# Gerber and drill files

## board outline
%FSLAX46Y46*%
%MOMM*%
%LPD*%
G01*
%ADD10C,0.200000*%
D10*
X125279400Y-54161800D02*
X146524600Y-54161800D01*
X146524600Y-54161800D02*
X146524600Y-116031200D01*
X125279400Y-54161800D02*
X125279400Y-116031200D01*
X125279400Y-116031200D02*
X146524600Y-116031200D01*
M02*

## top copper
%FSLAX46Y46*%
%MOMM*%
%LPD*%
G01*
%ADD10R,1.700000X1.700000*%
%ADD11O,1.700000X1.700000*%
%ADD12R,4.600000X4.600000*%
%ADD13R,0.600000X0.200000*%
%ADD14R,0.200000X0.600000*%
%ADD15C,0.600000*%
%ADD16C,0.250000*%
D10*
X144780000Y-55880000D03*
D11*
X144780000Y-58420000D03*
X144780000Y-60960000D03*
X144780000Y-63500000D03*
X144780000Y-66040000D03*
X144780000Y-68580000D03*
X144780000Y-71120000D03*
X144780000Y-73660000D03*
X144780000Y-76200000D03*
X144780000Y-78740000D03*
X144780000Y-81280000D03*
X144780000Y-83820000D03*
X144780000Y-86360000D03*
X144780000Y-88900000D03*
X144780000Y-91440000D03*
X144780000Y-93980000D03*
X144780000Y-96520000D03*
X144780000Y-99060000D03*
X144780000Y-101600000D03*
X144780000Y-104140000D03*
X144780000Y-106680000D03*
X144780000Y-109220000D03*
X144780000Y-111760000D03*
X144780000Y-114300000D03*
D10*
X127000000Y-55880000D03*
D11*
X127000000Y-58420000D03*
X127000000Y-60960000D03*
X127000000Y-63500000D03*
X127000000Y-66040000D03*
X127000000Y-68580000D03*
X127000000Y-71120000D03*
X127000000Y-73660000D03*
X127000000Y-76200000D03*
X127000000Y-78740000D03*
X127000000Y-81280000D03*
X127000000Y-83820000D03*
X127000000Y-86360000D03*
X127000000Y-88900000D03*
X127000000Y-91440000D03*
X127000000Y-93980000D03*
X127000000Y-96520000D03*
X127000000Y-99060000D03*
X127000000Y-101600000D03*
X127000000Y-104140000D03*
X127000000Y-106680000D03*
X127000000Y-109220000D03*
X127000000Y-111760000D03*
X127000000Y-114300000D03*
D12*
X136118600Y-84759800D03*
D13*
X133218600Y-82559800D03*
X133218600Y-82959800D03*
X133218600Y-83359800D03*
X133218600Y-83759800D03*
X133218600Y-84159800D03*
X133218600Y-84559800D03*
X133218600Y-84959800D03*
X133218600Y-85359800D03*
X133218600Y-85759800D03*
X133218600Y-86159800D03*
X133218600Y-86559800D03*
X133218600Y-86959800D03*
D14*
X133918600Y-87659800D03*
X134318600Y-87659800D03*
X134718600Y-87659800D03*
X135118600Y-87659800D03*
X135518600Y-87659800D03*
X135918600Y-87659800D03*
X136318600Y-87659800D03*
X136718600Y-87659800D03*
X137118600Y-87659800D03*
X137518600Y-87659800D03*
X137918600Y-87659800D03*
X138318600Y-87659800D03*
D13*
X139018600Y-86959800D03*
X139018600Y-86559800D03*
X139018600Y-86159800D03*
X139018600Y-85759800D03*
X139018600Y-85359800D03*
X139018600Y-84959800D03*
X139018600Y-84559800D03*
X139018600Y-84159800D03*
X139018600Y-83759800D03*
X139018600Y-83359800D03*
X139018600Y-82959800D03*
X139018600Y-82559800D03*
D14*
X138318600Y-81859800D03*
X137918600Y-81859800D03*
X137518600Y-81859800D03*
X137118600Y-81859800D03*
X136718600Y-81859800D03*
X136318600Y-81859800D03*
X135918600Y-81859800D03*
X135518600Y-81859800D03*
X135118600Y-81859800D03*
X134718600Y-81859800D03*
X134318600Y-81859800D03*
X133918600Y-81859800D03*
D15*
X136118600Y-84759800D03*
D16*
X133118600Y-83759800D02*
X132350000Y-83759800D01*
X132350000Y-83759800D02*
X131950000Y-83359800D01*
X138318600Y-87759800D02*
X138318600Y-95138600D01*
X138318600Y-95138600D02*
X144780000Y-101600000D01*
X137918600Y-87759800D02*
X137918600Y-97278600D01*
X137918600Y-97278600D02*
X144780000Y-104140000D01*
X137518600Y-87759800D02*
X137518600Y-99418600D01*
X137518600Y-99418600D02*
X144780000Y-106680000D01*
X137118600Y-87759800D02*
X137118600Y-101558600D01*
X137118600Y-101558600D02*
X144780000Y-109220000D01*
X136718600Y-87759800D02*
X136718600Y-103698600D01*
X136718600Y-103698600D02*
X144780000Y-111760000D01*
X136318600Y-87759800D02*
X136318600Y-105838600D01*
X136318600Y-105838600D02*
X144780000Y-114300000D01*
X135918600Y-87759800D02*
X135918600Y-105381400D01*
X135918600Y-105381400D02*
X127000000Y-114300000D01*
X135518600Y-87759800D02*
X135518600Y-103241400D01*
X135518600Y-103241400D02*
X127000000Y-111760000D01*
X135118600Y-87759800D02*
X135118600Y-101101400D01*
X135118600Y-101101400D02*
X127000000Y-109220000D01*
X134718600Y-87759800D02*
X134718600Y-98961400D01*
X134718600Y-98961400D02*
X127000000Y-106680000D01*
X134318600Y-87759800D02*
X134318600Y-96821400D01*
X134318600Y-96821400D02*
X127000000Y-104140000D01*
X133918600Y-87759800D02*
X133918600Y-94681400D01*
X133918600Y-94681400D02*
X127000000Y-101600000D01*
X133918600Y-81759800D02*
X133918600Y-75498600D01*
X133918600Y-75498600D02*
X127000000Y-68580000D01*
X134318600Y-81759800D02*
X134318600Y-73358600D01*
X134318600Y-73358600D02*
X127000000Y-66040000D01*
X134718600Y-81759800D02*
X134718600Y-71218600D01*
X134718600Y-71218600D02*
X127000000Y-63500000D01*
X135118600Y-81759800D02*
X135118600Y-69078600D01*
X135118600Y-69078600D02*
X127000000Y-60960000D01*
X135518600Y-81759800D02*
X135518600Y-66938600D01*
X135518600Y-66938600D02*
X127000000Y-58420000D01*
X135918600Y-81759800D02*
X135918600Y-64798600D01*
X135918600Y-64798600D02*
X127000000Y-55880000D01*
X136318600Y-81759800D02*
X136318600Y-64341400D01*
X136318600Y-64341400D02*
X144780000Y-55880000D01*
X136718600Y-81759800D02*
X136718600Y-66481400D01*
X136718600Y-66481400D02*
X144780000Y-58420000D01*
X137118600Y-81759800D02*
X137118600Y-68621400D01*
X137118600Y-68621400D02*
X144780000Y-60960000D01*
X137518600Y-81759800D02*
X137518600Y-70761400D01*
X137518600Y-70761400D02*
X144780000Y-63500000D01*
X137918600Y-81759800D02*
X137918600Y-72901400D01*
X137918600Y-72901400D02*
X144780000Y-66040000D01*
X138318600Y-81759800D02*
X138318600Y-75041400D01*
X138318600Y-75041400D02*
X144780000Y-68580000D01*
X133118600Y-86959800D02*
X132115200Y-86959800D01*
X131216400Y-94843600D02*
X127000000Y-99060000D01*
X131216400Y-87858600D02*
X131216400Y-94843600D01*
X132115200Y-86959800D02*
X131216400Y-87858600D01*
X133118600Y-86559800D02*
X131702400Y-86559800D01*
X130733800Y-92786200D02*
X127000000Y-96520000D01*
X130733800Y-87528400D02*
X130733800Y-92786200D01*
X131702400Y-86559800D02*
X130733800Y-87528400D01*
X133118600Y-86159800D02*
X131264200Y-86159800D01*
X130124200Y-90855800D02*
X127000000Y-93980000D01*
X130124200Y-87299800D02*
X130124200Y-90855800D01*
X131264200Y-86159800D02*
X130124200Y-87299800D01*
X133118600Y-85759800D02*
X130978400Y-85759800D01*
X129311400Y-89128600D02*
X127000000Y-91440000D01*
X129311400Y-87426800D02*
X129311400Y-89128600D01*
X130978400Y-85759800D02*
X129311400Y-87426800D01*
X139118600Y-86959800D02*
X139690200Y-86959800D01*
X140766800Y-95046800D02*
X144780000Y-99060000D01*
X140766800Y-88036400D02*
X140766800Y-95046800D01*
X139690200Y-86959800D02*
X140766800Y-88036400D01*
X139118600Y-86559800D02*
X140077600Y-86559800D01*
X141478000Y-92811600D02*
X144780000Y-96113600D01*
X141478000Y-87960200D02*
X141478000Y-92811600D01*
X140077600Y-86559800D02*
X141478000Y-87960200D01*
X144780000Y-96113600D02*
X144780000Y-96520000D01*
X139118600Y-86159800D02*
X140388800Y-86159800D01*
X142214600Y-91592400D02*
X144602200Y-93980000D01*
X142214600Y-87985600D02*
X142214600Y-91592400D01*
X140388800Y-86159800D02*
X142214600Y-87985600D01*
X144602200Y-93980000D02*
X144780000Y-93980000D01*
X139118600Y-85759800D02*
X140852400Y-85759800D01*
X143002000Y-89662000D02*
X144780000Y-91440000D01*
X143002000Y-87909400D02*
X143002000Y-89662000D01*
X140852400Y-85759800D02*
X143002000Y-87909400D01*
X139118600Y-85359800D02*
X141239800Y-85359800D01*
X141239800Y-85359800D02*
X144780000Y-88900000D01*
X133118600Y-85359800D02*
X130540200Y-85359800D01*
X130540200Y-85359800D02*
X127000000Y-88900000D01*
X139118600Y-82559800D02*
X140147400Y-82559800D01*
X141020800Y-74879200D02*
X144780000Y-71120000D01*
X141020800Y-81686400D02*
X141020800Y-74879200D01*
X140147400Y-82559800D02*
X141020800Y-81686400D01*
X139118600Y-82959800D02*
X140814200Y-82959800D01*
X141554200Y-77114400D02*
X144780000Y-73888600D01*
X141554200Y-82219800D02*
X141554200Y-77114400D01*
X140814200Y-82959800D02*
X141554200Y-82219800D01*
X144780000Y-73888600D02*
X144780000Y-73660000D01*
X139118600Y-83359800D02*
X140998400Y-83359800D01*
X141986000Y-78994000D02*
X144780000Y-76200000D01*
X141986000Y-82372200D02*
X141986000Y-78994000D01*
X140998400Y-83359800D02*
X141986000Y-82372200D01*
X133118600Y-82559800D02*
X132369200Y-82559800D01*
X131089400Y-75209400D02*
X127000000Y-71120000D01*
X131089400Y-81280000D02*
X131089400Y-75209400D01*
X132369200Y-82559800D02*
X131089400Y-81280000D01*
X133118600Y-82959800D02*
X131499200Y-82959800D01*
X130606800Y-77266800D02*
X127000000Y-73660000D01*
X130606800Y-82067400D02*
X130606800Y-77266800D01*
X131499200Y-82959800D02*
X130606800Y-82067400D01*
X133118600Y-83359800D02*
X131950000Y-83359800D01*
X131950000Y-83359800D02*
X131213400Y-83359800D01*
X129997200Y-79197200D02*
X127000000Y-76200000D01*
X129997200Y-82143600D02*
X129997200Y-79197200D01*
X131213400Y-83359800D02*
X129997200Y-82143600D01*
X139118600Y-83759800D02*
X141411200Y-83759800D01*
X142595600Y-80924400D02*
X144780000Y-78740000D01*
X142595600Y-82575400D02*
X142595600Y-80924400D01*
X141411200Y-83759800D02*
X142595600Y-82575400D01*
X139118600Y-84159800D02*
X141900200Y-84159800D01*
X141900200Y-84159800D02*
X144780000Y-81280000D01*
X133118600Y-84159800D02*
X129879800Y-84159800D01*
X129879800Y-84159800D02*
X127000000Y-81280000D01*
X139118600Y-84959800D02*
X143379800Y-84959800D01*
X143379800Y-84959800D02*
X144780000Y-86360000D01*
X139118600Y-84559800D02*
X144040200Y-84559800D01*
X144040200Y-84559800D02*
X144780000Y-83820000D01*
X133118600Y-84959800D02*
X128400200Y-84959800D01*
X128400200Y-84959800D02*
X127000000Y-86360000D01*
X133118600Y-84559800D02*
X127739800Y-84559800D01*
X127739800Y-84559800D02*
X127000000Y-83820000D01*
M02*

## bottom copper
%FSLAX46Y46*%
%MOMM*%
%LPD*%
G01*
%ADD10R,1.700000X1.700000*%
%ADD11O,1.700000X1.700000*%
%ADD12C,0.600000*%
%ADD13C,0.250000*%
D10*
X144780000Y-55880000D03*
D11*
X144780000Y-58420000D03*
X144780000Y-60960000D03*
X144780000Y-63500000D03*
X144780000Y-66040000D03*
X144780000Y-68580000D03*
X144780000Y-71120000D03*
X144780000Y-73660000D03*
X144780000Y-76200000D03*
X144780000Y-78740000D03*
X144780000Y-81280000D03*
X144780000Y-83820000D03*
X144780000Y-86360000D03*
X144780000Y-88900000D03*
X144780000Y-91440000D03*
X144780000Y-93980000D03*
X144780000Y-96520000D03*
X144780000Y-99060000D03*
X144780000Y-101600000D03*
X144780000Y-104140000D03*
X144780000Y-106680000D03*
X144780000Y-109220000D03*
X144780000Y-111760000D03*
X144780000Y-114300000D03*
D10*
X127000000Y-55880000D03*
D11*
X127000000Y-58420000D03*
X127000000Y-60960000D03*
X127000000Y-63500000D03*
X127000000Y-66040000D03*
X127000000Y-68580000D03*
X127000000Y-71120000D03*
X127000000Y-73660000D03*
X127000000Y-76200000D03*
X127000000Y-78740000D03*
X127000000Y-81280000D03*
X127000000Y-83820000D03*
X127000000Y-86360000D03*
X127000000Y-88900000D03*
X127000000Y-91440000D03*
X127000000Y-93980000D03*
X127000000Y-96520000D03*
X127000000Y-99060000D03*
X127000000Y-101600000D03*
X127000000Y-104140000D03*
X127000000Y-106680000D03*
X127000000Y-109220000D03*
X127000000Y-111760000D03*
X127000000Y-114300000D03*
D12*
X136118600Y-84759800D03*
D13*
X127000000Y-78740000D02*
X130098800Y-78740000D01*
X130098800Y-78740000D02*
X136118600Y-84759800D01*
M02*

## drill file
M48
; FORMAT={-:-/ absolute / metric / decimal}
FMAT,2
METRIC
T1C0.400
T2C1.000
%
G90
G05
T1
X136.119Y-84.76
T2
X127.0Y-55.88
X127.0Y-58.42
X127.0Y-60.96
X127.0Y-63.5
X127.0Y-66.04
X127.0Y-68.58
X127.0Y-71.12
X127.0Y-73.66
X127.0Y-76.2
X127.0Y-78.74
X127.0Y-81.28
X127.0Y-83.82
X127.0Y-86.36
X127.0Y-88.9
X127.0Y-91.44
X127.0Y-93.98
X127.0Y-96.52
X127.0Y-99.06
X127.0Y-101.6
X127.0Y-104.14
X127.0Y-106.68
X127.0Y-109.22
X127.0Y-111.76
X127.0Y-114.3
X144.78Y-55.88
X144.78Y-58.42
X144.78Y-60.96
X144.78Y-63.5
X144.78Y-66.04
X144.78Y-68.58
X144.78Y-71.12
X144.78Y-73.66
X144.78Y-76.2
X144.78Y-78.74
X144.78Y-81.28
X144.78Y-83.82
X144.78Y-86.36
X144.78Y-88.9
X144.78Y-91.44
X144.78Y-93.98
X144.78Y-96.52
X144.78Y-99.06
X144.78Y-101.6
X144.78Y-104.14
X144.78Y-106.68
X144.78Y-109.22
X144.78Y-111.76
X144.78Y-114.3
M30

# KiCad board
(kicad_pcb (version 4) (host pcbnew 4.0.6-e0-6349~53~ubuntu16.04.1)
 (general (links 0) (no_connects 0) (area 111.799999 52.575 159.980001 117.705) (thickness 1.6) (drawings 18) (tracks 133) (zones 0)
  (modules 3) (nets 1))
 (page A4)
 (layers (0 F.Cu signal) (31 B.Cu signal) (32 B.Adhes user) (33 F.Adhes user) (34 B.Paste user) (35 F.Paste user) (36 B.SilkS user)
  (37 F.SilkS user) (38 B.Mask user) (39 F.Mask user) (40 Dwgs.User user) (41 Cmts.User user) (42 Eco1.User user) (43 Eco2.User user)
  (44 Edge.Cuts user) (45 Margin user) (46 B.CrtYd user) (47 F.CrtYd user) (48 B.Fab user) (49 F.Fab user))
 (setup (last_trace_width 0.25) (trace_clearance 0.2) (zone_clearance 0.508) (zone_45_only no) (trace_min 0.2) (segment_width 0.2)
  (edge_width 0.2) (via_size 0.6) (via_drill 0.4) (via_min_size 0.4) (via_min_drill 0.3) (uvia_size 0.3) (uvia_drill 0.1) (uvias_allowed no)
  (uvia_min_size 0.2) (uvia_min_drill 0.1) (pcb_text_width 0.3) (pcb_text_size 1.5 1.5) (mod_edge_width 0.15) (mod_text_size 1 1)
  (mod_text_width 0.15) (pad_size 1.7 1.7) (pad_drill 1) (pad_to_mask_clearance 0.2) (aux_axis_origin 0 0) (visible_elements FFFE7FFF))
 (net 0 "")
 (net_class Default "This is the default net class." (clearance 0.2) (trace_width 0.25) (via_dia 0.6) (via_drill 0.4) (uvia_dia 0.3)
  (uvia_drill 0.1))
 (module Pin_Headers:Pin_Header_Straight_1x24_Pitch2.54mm (layer F.Cu) (at 144.78 55.88)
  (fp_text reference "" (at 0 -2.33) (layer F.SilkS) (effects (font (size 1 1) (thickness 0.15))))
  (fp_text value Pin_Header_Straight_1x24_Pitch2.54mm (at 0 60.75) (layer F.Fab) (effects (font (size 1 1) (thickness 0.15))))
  (pad 1 thru_hole rect (at 0 0) (size 1.7 1.7) (drill 1) (layers *.Cu *.Mask))
  (pad 2 thru_hole oval (at 0 2.54) (size 1.7 1.7) (drill 1) (layers *.Cu *.Mask))
  (pad 3 thru_hole oval (at 0 5.08) (size 1.7 1.7) (drill 1) (layers *.Cu *.Mask))
  (pad 4 thru_hole oval (at 0 7.62) (size 1.7 1.7) (drill 1) (layers *.Cu *.Mask))
  (pad 5 thru_hole oval (at 0 10.16) (size 1.7 1.7) (drill 1) (layers *.Cu *.Mask))
  (pad 6 thru_hole oval (at 0 12.7) (size 1.7 1.7) (drill 1) (layers *.Cu *.Mask))
  (pad 7 thru_hole oval (at 0 15.24) (size 1.7 1.7) (drill 1) (layers *.Cu *.Mask))
  (pad 8 thru_hole oval (at 0 17.78) (size 1.7 1.7) (drill 1) (layers *.Cu *.Mask))
  (pad 9 thru_hole oval (at 0 20.32) (size 1.7 1.7) (drill 1) (layers *.Cu *.Mask))
  (pad 10 thru_hole oval (at 0 22.86) (size 1.7 1.7) (drill 1) (layers *.Cu *.Mask))
  (pad 11 thru_hole oval (at 0 25.4) (size 1.7 1.7) (drill 1) (layers *.Cu *.Mask))
  (pad 12 thru_hole oval (at 0 27.94) (size 1.7 1.7) (drill 1) (layers *.Cu *.Mask))
  (pad 13 thru_hole oval (at 0 30.48) (size 1.7 1.7) (drill 1) (layers *.Cu *.Mask))
  (pad 14 thru_hole oval (at 0 33.02) (size 1.7 1.7) (drill 1) (layers *.Cu *.Mask))
  (pad 15 thru_hole oval (at 0 35.56) (size 1.7 1.7) (drill 1) (layers *.Cu *.Mask))
  (pad 16 thru_hole oval (at 0 38.1) (size 1.7 1.7) (drill 1) (layers *.Cu *.Mask))
  (pad 17 thru_hole oval (at 0 40.64) (size 1.7 1.7) (drill 1) (layers *.Cu *.Mask))
  (pad 18 thru_hole oval (at 0 43.18) (size 1.7 1.7) (drill 1) (layers *.Cu *.Mask))
  (pad 19 thru_hole oval (at 0 45.72) (size 1.7 1.7) (drill 1) (layers *.Cu *.Mask))
  (pad 20 thru_hole oval (at 0 48.26) (size 1.7 1.7) (drill 1) (layers *.Cu *.Mask))
  (pad 21 thru_hole oval (at 0 50.8) (size 1.7 1.7) (drill 1) (layers *.Cu *.Mask))
  (pad 22 thru_hole oval (at 0 53.34) (size 1.7 1.7) (drill 1) (layers *.Cu *.Mask))
  (pad 23 thru_hole oval (at 0 55.88) (size 1.7 1.7) (drill 1) (layers *.Cu *.Mask))
  (pad 24 thru_hole oval (at 0 58.42) (size 1.7 1.7) (drill 1) (layers *.Cu *.Mask)))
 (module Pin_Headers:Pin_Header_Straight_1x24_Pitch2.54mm (layer F.Cu) (at 127 55.88)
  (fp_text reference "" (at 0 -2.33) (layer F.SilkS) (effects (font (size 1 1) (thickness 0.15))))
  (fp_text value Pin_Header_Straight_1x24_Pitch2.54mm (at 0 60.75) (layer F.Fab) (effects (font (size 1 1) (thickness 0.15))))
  (pad 1 thru_hole rect (at 0 0) (size 1.7 1.7) (drill 1) (layers *.Cu *.Mask))
  (pad 2 thru_hole oval (at 0 2.54) (size 1.7 1.7) (drill 1) (layers *.Cu *.Mask))
  (pad 3 thru_hole oval (at 0 5.08) (size 1.7 1.7) (drill 1) (layers *.Cu *.Mask))
  (pad 4 thru_hole oval (at 0 7.62) (size 1.7 1.7) (drill 1) (layers *.Cu *.Mask))
  (pad 5 thru_hole oval (at 0 10.16) (size 1.7 1.7) (drill 1) (layers *.Cu *.Mask))
  (pad 6 thru_hole oval (at 0 12.7) (size 1.7 1.7) (drill 1) (layers *.Cu *.Mask))
  (pad 7 thru_hole oval (at 0 15.24) (size 1.7 1.7) (drill 1) (layers *.Cu *.Mask))
  (pad 8 thru_hole oval (at 0 17.78) (size 1.7 1.7) (drill 1) (layers *.Cu *.Mask))
  (pad 9 thru_hole oval (at 0 20.32) (size 1.7 1.7) (drill 1) (layers *.Cu *.Mask))
  (pad 10 thru_hole oval (at 0 22.86) (size 1.7 1.7) (drill 1) (layers *.Cu *.Mask))
  (pad 11 thru_hole oval (at 0 25.4) (size 1.7 1.7) (drill 1) (layers *.Cu *.Mask))
  (pad 12 thru_hole oval (at 0 27.94) (size 1.7 1.7) (drill 1) (layers *.Cu *.Mask))
  (pad 13 thru_hole oval (at 0 30.48) (size 1.7 1.7) (drill 1) (layers *.Cu *.Mask))
  (pad 14 thru_hole oval (at 0 33.02) (size 1.7 1.7) (drill 1) (layers *.Cu *.Mask))
  (pad 15 thru_hole oval (at 0 35.56) (size 1.7 1.7) (drill 1) (layers *.Cu *.Mask))
  (pad 16 thru_hole oval (at 0 38.1) (size 1.7 1.7) (drill 1) (layers *.Cu *.Mask))
  (pad 17 thru_hole oval (at 0 40.64) (size 1.7 1.7) (drill 1) (layers *.Cu *.Mask))
  (pad 18 thru_hole oval (at 0 43.18) (size 1.7 1.7) (drill 1) (layers *.Cu *.Mask))
  (pad 19 thru_hole oval (at 0 45.72) (size 1.7 1.7) (drill 1) (layers *.Cu *.Mask))
  (pad 20 thru_hole oval (at 0 48.26) (size 1.7 1.7) (drill 1) (layers *.Cu *.Mask))
  (pad 21 thru_hole oval (at 0 50.8) (size 1.7 1.7) (drill 1) (layers *.Cu *.Mask))
  (pad 22 thru_hole oval (at 0 53.34) (size 1.7 1.7) (drill 1) (layers *.Cu *.Mask))
  (pad 23 thru_hole oval (at 0 55.88) (size 1.7 1.7) (drill 1) (layers *.Cu *.Mask))
  (pad 24 thru_hole oval (at 0 58.42) (size 1.7 1.7) (drill 1) (layers *.Cu *.Mask)))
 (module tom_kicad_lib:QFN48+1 (layer F.Cu) (at 136.1186 84.7598) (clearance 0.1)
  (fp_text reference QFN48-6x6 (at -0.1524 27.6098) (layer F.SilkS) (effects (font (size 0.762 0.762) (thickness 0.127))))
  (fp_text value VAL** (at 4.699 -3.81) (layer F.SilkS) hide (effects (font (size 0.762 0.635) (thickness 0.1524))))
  (pad 49 smd rect (at 0 0) (size 4.6 4.6) (layers F.Cu F.Paste F.Mask))
  (pad 1 smd rect (at -3 -2.2) (size 0.6 0.2) (drill (offset 0.1 0)) (layers F.Cu F.Paste F.Mask))
  (pad 2 smd rect (at -3 -1.8) (size 0.6 0.2) (drill (offset 0.1 0)) (layers F.Cu F.Paste F.Mask))
  (pad 3 smd rect (at -3 -1.4) (size 0.6 0.2) (drill (offset 0.1 0)) (layers F.Cu F.Paste F.Mask))
  (pad 4 smd rect (at -3 -1) (size 0.6 0.2) (drill (offset 0.1 0)) (layers F.Cu F.Paste F.Mask))
  (pad 5 smd rect (at -3 -0.6) (size 0.6 0.2) (drill (offset 0.1 0)) (layers F.Cu F.Paste F.Mask))
  (pad 6 smd rect (at -3 -0.2) (size 0.6 0.2) (drill (offset 0.1 0)) (layers F.Cu F.Paste F.Mask))
  (pad 7 smd rect (at -3 0.2) (size 0.6 0.2) (drill (offset 0.1 0)) (layers F.Cu F.Paste F.Mask))
  (pad 8 smd rect (at -3 0.6) (size 0.6 0.2) (drill (offset 0.1 0)) (layers F.Cu F.Paste F.Mask))
  (pad 9 smd rect (at -3 1) (size 0.6 0.2) (drill (offset 0.1 0)) (layers F.Cu F.Paste F.Mask))
  (pad 10 smd rect (at -3 1.4) (size 0.6 0.2) (drill (offset 0.1 0)) (layers F.Cu F.Paste F.Mask))
  (pad 11 smd rect (at -3 1.8) (size 0.6 0.2) (drill (offset 0.1 0)) (layers F.Cu F.Paste F.Mask))
  (pad 12 smd rect (at -3 2.2) (size 0.6 0.2) (drill (offset 0.1 0)) (layers F.Cu F.Paste F.Mask))
  (pad 13 smd rect (at -2.2 3 90) (size 0.6 0.2) (drill (offset 0.1 0)) (layers F.Cu F.Paste F.Mask))
  (pad 14 smd rect (at -1.8 3 90) (size 0.6 0.2) (drill (offset 0.1 0)) (layers F.Cu F.Paste F.Mask))
  (pad 15 smd rect (at -1.4 3 90) (size 0.6 0.2) (drill (offset 0.1 0)) (layers F.Cu F.Paste F.Mask))
  (pad 16 smd rect (at -1 3 90) (size 0.6 0.2) (drill (offset 0.1 0)) (layers F.Cu F.Paste F.Mask))
  (pad 17 smd rect (at -0.6 3 90) (size 0.6 0.2) (drill (offset 0.1 0)) (layers F.Cu F.Paste F.Mask))
  (pad 18 smd rect (at -0.2 3 90) (size 0.6 0.2) (drill (offset 0.1 0)) (layers F.Cu F.Paste F.Mask))
  (pad 19 smd rect (at 0.2 3 90) (size 0.6 0.2) (drill (offset 0.1 0)) (layers F.Cu F.Paste F.Mask))
  (pad 20 smd rect (at 0.6 3 90) (size 0.6 0.2) (drill (offset 0.1 0)) (layers F.Cu F.Paste F.Mask))
  (pad 21 smd rect (at 1 3 90) (size 0.6 0.2) (drill (offset 0.1 0)) (layers F.Cu F.Paste F.Mask))
  (pad 22 smd rect (at 1.4 3 90) (size 0.6 0.2) (drill (offset 0.1 0)) (layers F.Cu F.Paste F.Mask))
  (pad 23 smd rect (at 1.8 3 90) (size 0.6 0.2) (drill (offset 0.1 0)) (layers F.Cu F.Paste F.Mask))
  (pad 24 smd rect (at 2.2 3 90) (size 0.6 0.2) (drill (offset 0.1 0)) (layers F.Cu F.Paste F.Mask))
  (pad 25 smd rect (at 3 2.2 180) (size 0.6 0.2) (drill (offset 0.1 0)) (layers F.Cu F.Paste F.Mask))
  (pad 26 smd rect (at 3 1.8 180) (size 0.6 0.2) (drill (offset 0.1 0)) (layers F.Cu F.Paste F.Mask))
  (pad 27 smd rect (at 3 1.4 180) (size 0.6 0.2) (drill (offset 0.1 0)) (layers F.Cu F.Paste F.Mask))
  (pad 28 smd rect (at 3 1 180) (size 0.6 0.2) (drill (offset 0.1 0)) (layers F.Cu F.Paste F.Mask))
  (pad 29 smd rect (at 3 0.6 180) (size 0.6 0.2) (drill (offset 0.1 0)) (layers F.Cu F.Paste F.Mask))
  (pad 30 smd rect (at 3 0.2 180) (size 0.6 0.2) (drill (offset 0.1 0)) (layers F.Cu F.Paste F.Mask))
  (pad 31 smd rect (at 3 -0.2 180) (size 0.6 0.2) (drill (offset 0.1 0)) (layers F.Cu F.Paste F.Mask))
  (pad 32 smd rect (at 3 -0.6 180) (size 0.6 0.2) (drill (offset 0.1 0)) (layers F.Cu F.Paste F.Mask))
  (pad 33 smd rect (at 3 -1 180) (size 0.6 0.2) (drill (offset 0.1 0)) (layers F.Cu F.Paste F.Mask))
  (pad 34 smd rect (at 3 -1.4 180) (size 0.6 0.2) (drill (offset 0.1 0)) (layers F.Cu F.Paste F.Mask))
  (pad 35 smd rect (at 3 -1.8 180) (size 0.6 0.2) (drill (offset 0.1 0)) (layers F.Cu F.Paste F.Mask))
  (pad 36 smd rect (at 3 -2.2 180) (size 0.6 0.2) (drill (offset 0.1 0)) (layers F.Cu F.Paste F.Mask))
  (pad 37 smd rect (at 2.2 -3 270) (size 0.6 0.2) (drill (offset 0.1 0)) (layers F.Cu F.Paste F.Mask))
  (pad 38 smd rect (at 1.8 -3 270) (size 0.6 0.2) (drill (offset 0.1 0)) (layers F.Cu F.Paste F.Mask))
  (pad 39 smd rect (at 1.4 -3 270) (size 0.6 0.2) (drill (offset 0.1 0)) (layers F.Cu F.Paste F.Mask))
  (pad 40 smd rect (at 1 -3 270) (size 0.6 0.2) (drill (offset 0.1 0)) (layers F.Cu F.Paste F.Mask))
  (pad 41 smd rect (at 0.6 -3 270) (size 0.6 0.2) (drill (offset 0.1 0)) (layers F.Cu F.Paste F.Mask))
  (pad 42 smd rect (at 0.2 -3 270) (size 0.6 0.2) (drill (offset 0.1 0)) (layers F.Cu F.Paste F.Mask))
  (pad 43 smd rect (at -0.2 -3 270) (size 0.6 0.2) (drill (offset 0.1 0)) (layers F.Cu F.Paste F.Mask))
  (pad 44 smd rect (at -0.6 -3 270) (size 0.6 0.2) (drill (offset 0.1 0)) (layers F.Cu F.Paste F.Mask))
  (pad 45 smd rect (at -1 -3 270) (size 0.6 0.2) (drill (offset 0.1 0)) (layers F.Cu F.Paste F.Mask))
  (pad 46 smd rect (at -1.4 -3 270) (size 0.6 0.2) (drill (offset 0.1 0)) (layers F.Cu F.Paste F.Mask))
  (pad 47 smd rect (at -1.8 -3 270) (size 0.6 0.2) (drill (offset 0.1 0)) (layers F.Cu F.Paste F.Mask))
  (pad 48 smd rect (at -2.2 -3 270) (size 0.6 0.2) (drill (offset 0.1 0)) (layers F.Cu F.Paste F.Mask)))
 (gr_line (start 125.2794 54.1618) (end 146.5246 54.1618) (angle 90) (layer Edge.Cuts) (width 0.2))
 (gr_line (start 146.5246 54.1618) (end 146.5246 116.0312) (angle 90) (layer Edge.Cuts) (width 0.2))
 (gr_line (start 125.2794 54.1618) (end 125.2794 116.0312) (angle 90) (layer Edge.Cuts) (width 0.2))
 (gr_line (start 125.2794 116.0312) (end 146.5246 116.0312) (angle 90) (layer Edge.Cuts) (width 0.2))
 (via (at 136.1186 84.7598) (size 0.6) (drill 0.4) (layers F.Cu B.Cu) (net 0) (status C00000))
 (segment (start 127 78.74) (end 130.0988 78.74) (width 0.25) (layer B.Cu) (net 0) (status 400000))
 (segment (start 130.0988 78.74) (end 136.1186 84.7598) (width 0.25) (layer B.Cu) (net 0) (status 800000))
 (segment (start 133.1186 83.7598) (end 132.35 83.7598) (width 0.25) (layer F.Cu) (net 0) (status 400000))
 (segment (start 132.35 83.7598) (end 131.95 83.3598) (width 0.25) (layer F.Cu) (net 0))
 (segment (start 138.3186 87.7598) (end 138.3186 95.1386) (width 0.25) (layer F.Cu) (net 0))
 (segment (start 138.3186 95.1386) (end 144.78 101.6) (width 0.25) (layer F.Cu) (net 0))
 (segment (start 137.9186 87.7598) (end 137.9186 97.2786) (width 0.25) (layer F.Cu) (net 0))
 (segment (start 137.9186 97.2786) (end 144.78 104.14) (width 0.25) (layer F.Cu) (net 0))
 (segment (start 137.5186 87.7598) (end 137.5186 99.4186) (width 0.25) (layer F.Cu) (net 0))
 (segment (start 137.5186 99.4186) (end 144.78 106.68) (width 0.25) (layer F.Cu) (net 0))
 (segment (start 137.1186 87.7598) (end 137.1186 101.5586) (width 0.25) (layer F.Cu) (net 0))
 (segment (start 137.1186 101.5586) (end 144.78 109.22) (width 0.25) (layer F.Cu) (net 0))
 (segment (start 136.7186 87.7598) (end 136.7186 103.6986) (width 0.25) (layer F.Cu) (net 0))
 (segment (start 136.7186 103.6986) (end 144.78 111.76) (width 0.25) (layer F.Cu) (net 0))
 (segment (start 136.3186 87.7598) (end 136.3186 105.8386) (width 0.25) (layer F.Cu) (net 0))
 (segment (start 136.3186 105.8386) (end 144.78 114.3) (width 0.25) (layer F.Cu) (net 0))
 (segment (start 135.9186 87.7598) (end 135.9186 105.3814) (width 0.25) (layer F.Cu) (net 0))
 (segment (start 135.9186 105.3814) (end 127 114.3) (width 0.25) (layer F.Cu) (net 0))
 (segment (start 135.5186 87.7598) (end 135.5186 103.2414) (width 0.25) (layer F.Cu) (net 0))
 (segment (start 135.5186 103.2414) (end 127 111.76) (width 0.25) (layer F.Cu) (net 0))
 (segment (start 135.1186 87.7598) (end 135.1186 101.1014) (width 0.25) (layer F.Cu) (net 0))
 (segment (start 135.1186 101.1014) (end 127 109.22) (width 0.25) (layer F.Cu) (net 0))
 (segment (start 134.7186 87.7598) (end 134.7186 98.9614) (width 0.25) (layer F.Cu) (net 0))
 (segment (start 134.7186 98.9614) (end 127 106.68) (width 0.25) (layer F.Cu) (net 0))
 (segment (start 134.3186 87.7598) (end 134.3186 96.8214) (width 0.25) (layer F.Cu) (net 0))
 (segment (start 134.3186 96.8214) (end 127 104.14) (width 0.25) (layer F.Cu) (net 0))
 (segment (start 133.9186 87.7598) (end 133.9186 94.6814) (width 0.25) (layer F.Cu) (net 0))
 (segment (start 133.9186 94.6814) (end 127 101.6) (width 0.25) (layer F.Cu) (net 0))
 (segment (start 133.9186 81.7598) (end 133.9186 75.4986) (width 0.25) (layer F.Cu) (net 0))
 (segment (start 133.9186 75.4986) (end 127 68.58) (width 0.25) (layer F.Cu) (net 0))
 (segment (start 134.3186 81.7598) (end 134.3186 73.3586) (width 0.25) (layer F.Cu) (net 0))
 (segment (start 134.3186 73.3586) (end 127 66.04) (width 0.25) (layer F.Cu) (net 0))
 (segment (start 134.7186 81.7598) (end 134.7186 71.2186) (width 0.25) (layer F.Cu) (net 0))
 (segment (start 134.7186 71.2186) (end 127 63.5) (width 0.25) (layer F.Cu) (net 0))
 (segment (start 135.1186 81.7598) (end 135.1186 69.0786) (width 0.25) (layer F.Cu) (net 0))
 (segment (start 135.1186 69.0786) (end 127 60.96) (width 0.25) (layer F.Cu) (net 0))
 (segment (start 135.5186 81.7598) (end 135.5186 66.9386) (width 0.25) (layer F.Cu) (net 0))
 (segment (start 135.5186 66.9386) (end 127 58.42) (width 0.25) (layer F.Cu) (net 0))
 (segment (start 135.9186 81.7598) (end 135.9186 64.7986) (width 0.25) (layer F.Cu) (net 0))
 (segment (start 135.9186 64.7986) (end 127 55.88) (width 0.25) (layer F.Cu) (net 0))
 (segment (start 136.3186 81.7598) (end 136.3186 64.3414) (width 0.25) (layer F.Cu) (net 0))
 (segment (start 136.3186 64.3414) (end 144.78 55.88) (width 0.25) (layer F.Cu) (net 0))
 (segment (start 136.7186 81.7598) (end 136.7186 66.4814) (width 0.25) (layer F.Cu) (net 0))
 (segment (start 136.7186 66.4814) (end 144.78 58.42) (width 0.25) (layer F.Cu) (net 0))
 (segment (start 137.1186 81.7598) (end 137.1186 68.6214) (width 0.25) (layer F.Cu) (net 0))
 (segment (start 137.1186 68.6214) (end 144.78 60.96) (width 0.25) (layer F.Cu) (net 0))
 (segment (start 137.5186 81.7598) (end 137.5186 70.7614) (width 0.25) (layer F.Cu) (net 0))
 (segment (start 137.5186 70.7614) (end 144.78 63.5) (width 0.25) (layer F.Cu) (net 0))
 (segment (start 137.9186 81.7598) (end 137.9186 72.9014) (width 0.25) (layer F.Cu) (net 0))
 (segment (start 137.9186 72.9014) (end 144.78 66.04) (width 0.25) (layer F.Cu) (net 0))
 (segment (start 138.3186 81.7598) (end 138.3186 75.0414) (width 0.25) (layer F.Cu) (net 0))
 (segment (start 138.3186 75.0414) (end 144.78 68.58) (width 0.25) (layer F.Cu) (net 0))
 (segment (start 133.1186 86.9598) (end 132.1152 86.9598) (width 0.25) (layer F.Cu) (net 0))
 (segment (start 131.2164 94.8436) (end 127 99.06) (width 0.25) (layer F.Cu) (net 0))
 (segment (start 131.2164 87.8586) (end 131.2164 94.8436) (width 0.25) (layer F.Cu) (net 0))
 (segment (start 132.1152 86.9598) (end 131.2164 87.8586) (width 0.25) (layer F.Cu) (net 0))
 (segment (start 133.1186 86.5598) (end 131.7024 86.5598) (width 0.25) (layer F.Cu) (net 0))
 (segment (start 130.7338 92.7862) (end 127 96.52) (width 0.25) (layer F.Cu) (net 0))
 (segment (start 130.7338 87.5284) (end 130.7338 92.7862) (width 0.25) (layer F.Cu) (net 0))
 (segment (start 131.7024 86.5598) (end 130.7338 87.5284) (width 0.25) (layer F.Cu) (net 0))
 (segment (start 133.1186 86.1598) (end 131.2642 86.1598) (width 0.25) (layer F.Cu) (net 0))
 (segment (start 130.1242 90.8558) (end 127 93.98) (width 0.25) (layer F.Cu) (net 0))
 (segment (start 130.1242 87.2998) (end 130.1242 90.8558) (width 0.25) (layer F.Cu) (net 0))
 (segment (start 131.2642 86.1598) (end 130.1242 87.2998) (width 0.25) (layer F.Cu) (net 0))
 (segment (start 133.1186 85.7598) (end 130.9784 85.7598) (width 0.25) (layer F.Cu) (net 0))
 (segment (start 129.3114 89.1286) (end 127 91.44) (width 0.25) (layer F.Cu) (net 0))
 (segment (start 129.3114 87.4268) (end 129.3114 89.1286) (width 0.25) (layer F.Cu) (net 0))
 (segment (start 130.9784 85.7598) (end 129.3114 87.4268) (width 0.25) (layer F.Cu) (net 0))
 (segment (start 139.1186 86.9598) (end 139.6902 86.9598) (width 0.25) (layer F.Cu) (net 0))
 (segment (start 140.7668 95.0468) (end 144.78 99.06) (width 0.25) (layer F.Cu) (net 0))
 (segment (start 140.7668 88.0364) (end 140.7668 95.0468) (width 0.25) (layer F.Cu) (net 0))
 (segment (start 139.6902 86.9598) (end 140.7668 88.0364) (width 0.25) (layer F.Cu) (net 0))
 (segment (start 139.1186 86.5598) (end 140.0776 86.5598) (width 0.25) (layer F.Cu) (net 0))
 (segment (start 141.478 92.8116) (end 144.78 96.1136) (width 0.25) (layer F.Cu) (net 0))
 (segment (start 141.478 87.9602) (end 141.478 92.8116) (width 0.25) (layer F.Cu) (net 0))
 (segment (start 140.0776 86.5598) (end 141.478 87.9602) (width 0.25) (layer F.Cu) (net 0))
 (segment (start 144.78 96.1136) (end 144.78 96.52) (width 0.25) (layer F.Cu) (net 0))
 (segment (start 139.1186 86.1598) (end 140.3888 86.1598) (width 0.25) (layer F.Cu) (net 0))
 (segment (start 142.2146 91.5924) (end 144.6022 93.98) (width 0.25) (layer F.Cu) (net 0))
 (segment (start 142.2146 87.9856) (end 142.2146 91.5924) (width 0.25) (layer F.Cu) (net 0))
 (segment (start 140.3888 86.1598) (end 142.2146 87.9856) (width 0.25) (layer F.Cu) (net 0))
 (segment (start 144.6022 93.98) (end 144.78 93.98) (width 0.25) (layer F.Cu) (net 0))
 (segment (start 139.1186 85.7598) (end 140.8524 85.7598) (width 0.25) (layer F.Cu) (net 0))
 (segment (start 143.002 89.662) (end 144.78 91.44) (width 0.25) (layer F.Cu) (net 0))
 (segment (start 143.002 87.9094) (end 143.002 89.662) (width 0.25) (layer F.Cu) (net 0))
 (segment (start 140.8524 85.7598) (end 143.002 87.9094) (width 0.25) (layer F.Cu) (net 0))
 (segment (start 139.1186 85.3598) (end 141.2398 85.3598) (width 0.25) (layer F.Cu) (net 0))
 (segment (start 141.2398 85.3598) (end 144.78 88.9) (width 0.25) (layer F.Cu) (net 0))
 (segment (start 133.1186 85.3598) (end 130.5402 85.3598) (width 0.25) (layer F.Cu) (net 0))
 (segment (start 130.5402 85.3598) (end 127 88.9) (width 0.25) (layer F.Cu) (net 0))
 (segment (start 139.1186 82.5598) (end 140.1474 82.5598) (width 0.25) (layer F.Cu) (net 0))
 (segment (start 141.0208 74.8792) (end 144.78 71.12) (width 0.25) (layer F.Cu) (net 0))
 (segment (start 141.0208 81.6864) (end 141.0208 74.8792) (width 0.25) (layer F.Cu) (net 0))
 (segment (start 140.1474 82.5598) (end 141.0208 81.6864) (width 0.25) (layer F.Cu) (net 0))
 (segment (start 139.1186 82.9598) (end 140.8142 82.9598) (width 0.25) (layer F.Cu) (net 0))
 (segment (start 141.5542 77.1144) (end 144.78 73.8886) (width 0.25) (layer F.Cu) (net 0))
 (segment (start 141.5542 82.2198) (end 141.5542 77.1144) (width 0.25) (layer F.Cu) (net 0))
 (segment (start 140.8142 82.9598) (end 141.5542 82.2198) (width 0.25) (layer F.Cu) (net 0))
 (segment (start 144.78 73.8886) (end 144.78 73.66) (width 0.25) (layer F.Cu) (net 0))
 (segment (start 139.1186 83.3598) (end 140.9984 83.3598) (width 0.25) (layer F.Cu) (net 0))
 (segment (start 141.986 78.994) (end 144.78 76.2) (width 0.25) (layer F.Cu) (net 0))
 (segment (start 141.986 82.3722) (end 141.986 78.994) (width 0.25) (layer F.Cu) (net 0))
 (segment (start 140.9984 83.3598) (end 141.986 82.3722) (width 0.25) (layer F.Cu) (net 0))
 (segment (start 133.1186 82.5598) (end 132.3692 82.5598) (width 0.25) (layer F.Cu) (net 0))
 (segment (start 131.0894 75.2094) (end 127 71.12) (width 0.25) (layer F.Cu) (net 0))
 (segment (start 131.0894 81.28) (end 131.0894 75.2094) (width 0.25) (layer F.Cu) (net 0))
 (segment (start 132.3692 82.5598) (end 131.0894 81.28) (width 0.25) (layer F.Cu) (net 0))
 (segment (start 133.1186 82.9598) (end 131.4992 82.9598) (width 0.25) (layer F.Cu) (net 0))
 (segment (start 130.6068 77.2668) (end 127 73.66) (width 0.25) (layer F.Cu) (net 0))
 (segment (start 130.6068 82.0674) (end 130.6068 77.2668) (width 0.25) (layer F.Cu) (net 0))
 (segment (start 131.4992 82.9598) (end 130.6068 82.0674) (width 0.25) (layer F.Cu) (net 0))
 (segment (start 133.1186 83.3598) (end 131.95 83.3598) (width 0.25) (layer F.Cu) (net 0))
 (segment (start 131.95 83.3598) (end 131.2134 83.3598) (width 0.25) (layer F.Cu) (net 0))
 (segment (start 129.9972 79.1972) (end 127 76.2) (width 0.25) (layer F.Cu) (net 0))
 (segment (start 129.9972 82.1436) (end 129.9972 79.1972) (width 0.25) (layer F.Cu) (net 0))
 (segment (start 131.2134 83.3598) (end 129.9972 82.1436) (width 0.25) (layer F.Cu) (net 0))
 (segment (start 139.1186 83.7598) (end 141.4112 83.7598) (width 0.25) (layer F.Cu) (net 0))
 (segment (start 142.5956 80.9244) (end 144.78 78.74) (width 0.25) (layer F.Cu) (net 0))
 (segment (start 142.5956 82.5754) (end 142.5956 80.9244) (width 0.25) (layer F.Cu) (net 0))
 (segment (start 141.4112 83.7598) (end 142.5956 82.5754) (width 0.25) (layer F.Cu) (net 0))
 (segment (start 139.1186 84.1598) (end 141.9002 84.1598) (width 0.25) (layer F.Cu) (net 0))
 (segment (start 141.9002 84.1598) (end 144.78 81.28) (width 0.25) (layer F.Cu) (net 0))
 (segment (start 133.1186 84.1598) (end 129.8798 84.1598) (width 0.25) (layer F.Cu) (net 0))
 (segment (start 129.8798 84.1598) (end 127 81.28) (width 0.25) (layer F.Cu) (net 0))
 (segment (start 139.1186 84.9598) (end 143.3798 84.9598) (width 0.25) (layer F.Cu) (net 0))
 (segment (start 143.3798 84.9598) (end 144.78 86.36) (width 0.25) (layer F.Cu) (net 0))
 (segment (start 139.1186 84.5598) (end 144.0402 84.5598) (width 0.25) (layer F.Cu) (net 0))
 (segment (start 144.0402 84.5598) (end 144.78 83.82) (width 0.25) (layer F.Cu) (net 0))
 (segment (start 133.1186 84.9598) (end 128.4002 84.9598) (width 0.25) (layer F.Cu) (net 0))
 (segment (start 128.4002 84.9598) (end 127 86.36) (width 0.25) (layer F.Cu) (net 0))
 (segment (start 133.1186 84.5598) (end 127.7398 84.5598) (width 0.25) (layer F.Cu) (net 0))
 (segment (start 127.7398 84.5598) (end 127 83.82) (width 0.25) (layer F.Cu) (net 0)))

